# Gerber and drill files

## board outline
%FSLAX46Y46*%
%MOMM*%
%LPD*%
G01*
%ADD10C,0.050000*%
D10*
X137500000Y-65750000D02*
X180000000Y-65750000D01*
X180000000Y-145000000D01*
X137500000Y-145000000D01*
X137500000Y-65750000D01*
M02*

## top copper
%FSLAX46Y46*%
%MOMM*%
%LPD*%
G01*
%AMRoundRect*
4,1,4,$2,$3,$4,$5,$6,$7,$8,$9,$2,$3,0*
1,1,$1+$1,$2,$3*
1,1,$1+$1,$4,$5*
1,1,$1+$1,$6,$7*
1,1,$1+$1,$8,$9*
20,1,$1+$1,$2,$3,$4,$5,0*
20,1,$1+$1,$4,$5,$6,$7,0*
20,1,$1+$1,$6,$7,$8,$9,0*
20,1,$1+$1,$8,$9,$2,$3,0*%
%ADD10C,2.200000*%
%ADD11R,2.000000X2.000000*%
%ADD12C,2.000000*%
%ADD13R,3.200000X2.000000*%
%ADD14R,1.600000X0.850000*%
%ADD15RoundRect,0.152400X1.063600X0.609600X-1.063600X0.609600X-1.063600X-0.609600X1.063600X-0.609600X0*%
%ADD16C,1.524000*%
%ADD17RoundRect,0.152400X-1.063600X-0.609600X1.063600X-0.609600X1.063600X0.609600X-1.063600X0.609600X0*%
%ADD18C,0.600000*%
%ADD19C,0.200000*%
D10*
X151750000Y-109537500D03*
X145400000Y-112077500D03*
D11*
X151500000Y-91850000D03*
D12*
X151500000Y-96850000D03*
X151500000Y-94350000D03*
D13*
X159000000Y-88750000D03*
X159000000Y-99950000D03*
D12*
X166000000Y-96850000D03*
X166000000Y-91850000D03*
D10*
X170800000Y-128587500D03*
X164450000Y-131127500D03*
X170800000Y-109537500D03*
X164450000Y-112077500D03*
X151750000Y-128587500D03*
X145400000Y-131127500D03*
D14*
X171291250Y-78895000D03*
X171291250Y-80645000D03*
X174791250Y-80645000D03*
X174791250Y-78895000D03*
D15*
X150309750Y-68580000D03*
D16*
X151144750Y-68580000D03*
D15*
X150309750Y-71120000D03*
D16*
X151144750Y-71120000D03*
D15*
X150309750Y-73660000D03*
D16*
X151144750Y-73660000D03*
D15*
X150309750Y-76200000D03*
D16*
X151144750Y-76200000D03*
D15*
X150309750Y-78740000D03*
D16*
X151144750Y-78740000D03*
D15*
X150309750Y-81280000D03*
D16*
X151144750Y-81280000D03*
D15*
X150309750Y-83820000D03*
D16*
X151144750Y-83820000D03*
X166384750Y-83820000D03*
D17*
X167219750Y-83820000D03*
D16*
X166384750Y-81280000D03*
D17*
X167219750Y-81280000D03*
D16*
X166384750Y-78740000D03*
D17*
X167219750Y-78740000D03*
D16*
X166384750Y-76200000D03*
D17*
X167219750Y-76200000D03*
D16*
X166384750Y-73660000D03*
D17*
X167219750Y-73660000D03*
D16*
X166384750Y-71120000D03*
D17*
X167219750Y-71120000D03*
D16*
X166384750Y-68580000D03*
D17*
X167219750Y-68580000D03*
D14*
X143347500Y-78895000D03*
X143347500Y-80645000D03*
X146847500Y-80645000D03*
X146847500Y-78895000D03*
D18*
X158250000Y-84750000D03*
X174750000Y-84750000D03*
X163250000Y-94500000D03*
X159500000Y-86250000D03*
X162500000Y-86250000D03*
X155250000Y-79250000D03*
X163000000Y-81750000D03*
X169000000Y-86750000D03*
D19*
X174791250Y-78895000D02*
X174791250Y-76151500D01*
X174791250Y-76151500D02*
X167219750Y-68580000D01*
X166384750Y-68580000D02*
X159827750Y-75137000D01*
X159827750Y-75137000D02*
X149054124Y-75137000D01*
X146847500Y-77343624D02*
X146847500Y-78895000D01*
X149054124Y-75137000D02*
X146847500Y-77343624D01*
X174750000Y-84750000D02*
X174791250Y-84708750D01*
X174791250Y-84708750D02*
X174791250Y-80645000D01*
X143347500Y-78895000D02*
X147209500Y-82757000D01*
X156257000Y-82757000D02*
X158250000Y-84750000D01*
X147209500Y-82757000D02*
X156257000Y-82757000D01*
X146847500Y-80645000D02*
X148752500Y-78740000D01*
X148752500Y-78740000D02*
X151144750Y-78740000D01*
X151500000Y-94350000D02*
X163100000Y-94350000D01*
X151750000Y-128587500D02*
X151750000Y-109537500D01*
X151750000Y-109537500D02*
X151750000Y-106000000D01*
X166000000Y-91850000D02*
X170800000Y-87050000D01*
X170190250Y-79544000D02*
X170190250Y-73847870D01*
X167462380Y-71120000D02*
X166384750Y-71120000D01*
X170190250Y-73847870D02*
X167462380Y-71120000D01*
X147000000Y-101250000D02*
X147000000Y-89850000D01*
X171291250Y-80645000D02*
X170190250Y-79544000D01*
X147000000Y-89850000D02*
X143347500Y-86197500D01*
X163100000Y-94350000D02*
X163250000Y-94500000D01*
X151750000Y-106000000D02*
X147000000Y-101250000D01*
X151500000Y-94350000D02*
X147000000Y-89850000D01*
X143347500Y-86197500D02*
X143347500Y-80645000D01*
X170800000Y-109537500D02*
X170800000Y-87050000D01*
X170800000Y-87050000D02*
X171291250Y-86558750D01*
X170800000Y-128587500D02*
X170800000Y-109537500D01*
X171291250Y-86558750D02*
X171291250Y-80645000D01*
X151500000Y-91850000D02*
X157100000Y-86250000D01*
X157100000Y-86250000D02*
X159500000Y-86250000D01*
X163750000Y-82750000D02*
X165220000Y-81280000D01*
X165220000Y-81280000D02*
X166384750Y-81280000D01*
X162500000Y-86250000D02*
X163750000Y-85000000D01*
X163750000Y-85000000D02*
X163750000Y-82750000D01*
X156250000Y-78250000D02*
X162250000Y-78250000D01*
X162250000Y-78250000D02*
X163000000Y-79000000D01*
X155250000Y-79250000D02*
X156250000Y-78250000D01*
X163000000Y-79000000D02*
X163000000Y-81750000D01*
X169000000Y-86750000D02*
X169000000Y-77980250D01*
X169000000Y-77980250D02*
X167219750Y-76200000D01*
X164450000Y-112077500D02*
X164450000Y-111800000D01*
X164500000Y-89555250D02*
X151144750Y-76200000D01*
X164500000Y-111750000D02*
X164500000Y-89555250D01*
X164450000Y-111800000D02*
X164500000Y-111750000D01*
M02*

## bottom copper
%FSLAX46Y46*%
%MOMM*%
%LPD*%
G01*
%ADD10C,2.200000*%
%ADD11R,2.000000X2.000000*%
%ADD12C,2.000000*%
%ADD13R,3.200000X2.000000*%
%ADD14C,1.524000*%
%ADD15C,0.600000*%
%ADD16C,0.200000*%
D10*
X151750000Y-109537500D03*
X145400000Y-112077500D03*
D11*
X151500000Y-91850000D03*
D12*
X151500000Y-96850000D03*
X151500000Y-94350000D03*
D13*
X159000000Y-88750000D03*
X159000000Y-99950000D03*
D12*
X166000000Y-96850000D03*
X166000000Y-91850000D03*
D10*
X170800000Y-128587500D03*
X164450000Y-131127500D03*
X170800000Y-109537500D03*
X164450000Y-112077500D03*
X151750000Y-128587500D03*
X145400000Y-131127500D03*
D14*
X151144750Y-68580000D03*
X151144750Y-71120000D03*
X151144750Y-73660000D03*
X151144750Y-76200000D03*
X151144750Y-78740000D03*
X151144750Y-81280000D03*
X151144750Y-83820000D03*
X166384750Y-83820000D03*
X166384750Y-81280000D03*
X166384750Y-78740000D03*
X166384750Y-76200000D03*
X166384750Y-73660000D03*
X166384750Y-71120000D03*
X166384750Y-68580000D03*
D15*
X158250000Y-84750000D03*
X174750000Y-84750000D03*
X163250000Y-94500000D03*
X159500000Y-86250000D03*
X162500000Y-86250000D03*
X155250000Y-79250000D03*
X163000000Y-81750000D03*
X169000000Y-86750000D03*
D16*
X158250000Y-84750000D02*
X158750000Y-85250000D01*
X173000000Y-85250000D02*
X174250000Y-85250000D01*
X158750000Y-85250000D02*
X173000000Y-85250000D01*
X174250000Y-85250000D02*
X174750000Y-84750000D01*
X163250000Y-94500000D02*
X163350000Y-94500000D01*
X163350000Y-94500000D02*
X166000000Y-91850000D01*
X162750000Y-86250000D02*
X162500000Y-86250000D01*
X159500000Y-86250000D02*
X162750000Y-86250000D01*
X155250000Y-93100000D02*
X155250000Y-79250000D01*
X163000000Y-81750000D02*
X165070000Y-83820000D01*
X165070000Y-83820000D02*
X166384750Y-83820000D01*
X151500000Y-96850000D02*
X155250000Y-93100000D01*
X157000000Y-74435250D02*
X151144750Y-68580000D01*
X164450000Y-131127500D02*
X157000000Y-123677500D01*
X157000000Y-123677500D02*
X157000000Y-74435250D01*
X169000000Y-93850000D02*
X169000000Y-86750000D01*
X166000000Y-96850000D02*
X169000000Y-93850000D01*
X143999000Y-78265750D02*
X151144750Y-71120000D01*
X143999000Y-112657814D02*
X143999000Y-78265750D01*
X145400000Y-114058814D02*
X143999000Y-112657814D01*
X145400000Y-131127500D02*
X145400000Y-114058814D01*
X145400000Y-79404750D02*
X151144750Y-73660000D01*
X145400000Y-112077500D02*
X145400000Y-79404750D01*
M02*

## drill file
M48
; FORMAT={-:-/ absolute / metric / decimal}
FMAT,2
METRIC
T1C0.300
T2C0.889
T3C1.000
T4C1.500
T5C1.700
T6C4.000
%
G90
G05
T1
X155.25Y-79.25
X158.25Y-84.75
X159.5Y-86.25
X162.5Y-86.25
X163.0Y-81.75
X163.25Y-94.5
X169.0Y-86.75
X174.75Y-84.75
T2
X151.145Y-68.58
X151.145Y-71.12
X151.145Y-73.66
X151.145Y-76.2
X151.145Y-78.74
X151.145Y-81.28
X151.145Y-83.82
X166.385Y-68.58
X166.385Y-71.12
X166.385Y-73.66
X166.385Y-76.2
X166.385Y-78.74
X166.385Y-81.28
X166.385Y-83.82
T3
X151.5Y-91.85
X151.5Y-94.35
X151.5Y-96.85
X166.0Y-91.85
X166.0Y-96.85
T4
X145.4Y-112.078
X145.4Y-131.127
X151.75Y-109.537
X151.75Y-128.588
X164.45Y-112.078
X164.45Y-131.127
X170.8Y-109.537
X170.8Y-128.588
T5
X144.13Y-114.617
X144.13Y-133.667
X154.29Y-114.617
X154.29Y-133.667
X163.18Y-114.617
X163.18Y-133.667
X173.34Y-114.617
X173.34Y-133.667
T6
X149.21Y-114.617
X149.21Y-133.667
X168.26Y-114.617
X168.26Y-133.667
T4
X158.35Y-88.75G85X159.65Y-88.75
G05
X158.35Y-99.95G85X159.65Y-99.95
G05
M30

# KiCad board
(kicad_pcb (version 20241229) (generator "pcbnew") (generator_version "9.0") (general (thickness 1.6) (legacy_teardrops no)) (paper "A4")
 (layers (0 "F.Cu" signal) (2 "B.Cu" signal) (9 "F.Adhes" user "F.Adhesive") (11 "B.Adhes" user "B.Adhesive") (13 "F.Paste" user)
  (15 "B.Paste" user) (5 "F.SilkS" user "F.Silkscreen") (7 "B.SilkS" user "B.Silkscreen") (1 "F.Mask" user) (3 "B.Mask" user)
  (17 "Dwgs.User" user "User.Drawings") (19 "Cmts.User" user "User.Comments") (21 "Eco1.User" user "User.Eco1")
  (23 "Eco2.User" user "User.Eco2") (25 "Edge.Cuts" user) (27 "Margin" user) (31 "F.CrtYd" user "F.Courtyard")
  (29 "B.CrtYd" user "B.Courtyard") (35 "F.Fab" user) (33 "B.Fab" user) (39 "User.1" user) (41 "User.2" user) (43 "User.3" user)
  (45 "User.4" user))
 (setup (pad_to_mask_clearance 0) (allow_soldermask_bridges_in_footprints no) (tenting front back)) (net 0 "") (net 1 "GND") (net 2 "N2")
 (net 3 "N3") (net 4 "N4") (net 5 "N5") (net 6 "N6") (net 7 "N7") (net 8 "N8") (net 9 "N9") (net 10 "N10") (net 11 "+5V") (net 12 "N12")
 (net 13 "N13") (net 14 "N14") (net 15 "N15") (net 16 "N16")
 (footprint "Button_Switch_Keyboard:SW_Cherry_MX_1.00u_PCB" (layer "F.Cu") (at 151.75 109.5375)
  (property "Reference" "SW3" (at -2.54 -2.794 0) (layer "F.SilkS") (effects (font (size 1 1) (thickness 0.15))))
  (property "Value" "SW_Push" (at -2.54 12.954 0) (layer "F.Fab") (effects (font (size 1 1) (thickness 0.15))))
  (pad "" np_thru_hole circle (at -7.62 5.08) (size 1.7 1.7) (drill 1.7) (layers "*.Cu" "*.Mask"))
  (pad "" np_thru_hole circle (at -2.54 5.08) (size 4 4) (drill 4) (layers "*.Cu" "*.Mask"))
  (pad "" np_thru_hole circle (at 2.54 5.08) (size 1.7 1.7) (drill 1.7) (layers "*.Cu" "*.Mask"))
  (pad "1" thru_hole circle (at 0 0) (size 2.2 2.2) (drill 1.5) (layers "*.Cu" "*.Mask") (remove_unused_layers no) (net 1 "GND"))
  (pad "2" thru_hole circle (at -6.35 2.54) (size 2.2 2.2) (drill 1.5) (layers "*.Cu" "*.Mask") (remove_unused_layers no) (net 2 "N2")))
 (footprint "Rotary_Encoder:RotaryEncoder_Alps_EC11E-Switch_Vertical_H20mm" (layer "F.Cu") (at 151.5 91.85)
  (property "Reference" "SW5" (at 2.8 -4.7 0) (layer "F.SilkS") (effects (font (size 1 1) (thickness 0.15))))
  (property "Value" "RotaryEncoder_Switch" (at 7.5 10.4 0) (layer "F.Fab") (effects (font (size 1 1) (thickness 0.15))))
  (pad "A" thru_hole rect (at 0 0) (size 2 2) (drill 1) (layers "*.Cu" "*.Mask") (remove_unused_layers no) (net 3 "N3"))
  (pad "B" thru_hole circle (at 0 5) (size 2 2) (drill 1) (layers "*.Cu" "*.Mask") (remove_unused_layers no) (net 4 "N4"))
  (pad "C" thru_hole circle (at 0 2.5) (size 2 2) (drill 1) (layers "*.Cu" "*.Mask") (remove_unused_layers no) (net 1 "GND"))
  (pad "MP" thru_hole rect (at 7.5 -3.1) (size 3.2 2) (drill oval 2.8 1.5) (layers "*.Cu" "*.Mask") (remove_unused_layers no))
  (pad "MP" thru_hole rect (at 7.5 8.1) (size 3.2 2) (drill oval 2.8 1.5) (layers "*.Cu" "*.Mask") (remove_unused_layers no))
  (pad "S1" thru_hole circle (at 14.5 5) (size 2 2) (drill 1) (layers "*.Cu" "*.Mask") (remove_unused_layers no) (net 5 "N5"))
  (pad "S2" thru_hole circle (at 14.5 0) (size 2 2) (drill 1) (layers "*.Cu" "*.Mask") (remove_unused_layers no) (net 1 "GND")))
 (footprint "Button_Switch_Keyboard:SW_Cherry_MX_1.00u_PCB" (layer "F.Cu") (at 170.8 128.5875)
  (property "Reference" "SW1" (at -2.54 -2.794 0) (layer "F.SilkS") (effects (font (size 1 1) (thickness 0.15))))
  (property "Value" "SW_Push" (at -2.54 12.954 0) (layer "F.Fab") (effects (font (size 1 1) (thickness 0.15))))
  (pad "" np_thru_hole circle (at -7.62 5.08) (size 1.7 1.7) (drill 1.7) (layers "*.Cu" "*.Mask"))
  (pad "" np_thru_hole circle (at -2.54 5.08) (size 4 4) (drill 4) (layers "*.Cu" "*.Mask"))
  (pad "" np_thru_hole circle (at 2.54 5.08) (size 1.7 1.7) (drill 1.7) (layers "*.Cu" "*.Mask"))
  (pad "1" thru_hole circle (at 0 0) (size 2.2 2.2) (drill 1.5) (layers "*.Cu" "*.Mask") (remove_unused_layers no) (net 1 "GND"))
  (pad "2" thru_hole circle (at -6.35 2.54) (size 2.2 2.2) (drill 1.5) (layers "*.Cu" "*.Mask") (remove_unused_layers no) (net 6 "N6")))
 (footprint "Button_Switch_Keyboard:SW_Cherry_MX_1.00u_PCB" (layer "F.Cu") (at 170.8 109.5375)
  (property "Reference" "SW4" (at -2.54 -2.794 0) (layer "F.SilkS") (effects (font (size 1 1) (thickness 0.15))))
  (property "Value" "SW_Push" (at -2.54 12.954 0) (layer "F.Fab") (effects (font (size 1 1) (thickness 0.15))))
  (pad "" np_thru_hole circle (at -7.62 5.08) (size 1.7 1.7) (drill 1.7) (layers "*.Cu" "*.Mask"))
  (pad "" np_thru_hole circle (at -2.54 5.08) (size 4 4) (drill 4) (layers "*.Cu" "*.Mask"))
  (pad "" np_thru_hole circle (at 2.54 5.08) (size 1.7 1.7) (drill 1.7) (layers "*.Cu" "*.Mask"))
  (pad "1" thru_hole circle (at 0 0) (size 2.2 2.2) (drill 1.5) (layers "*.Cu" "*.Mask") (remove_unused_layers no) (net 1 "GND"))
  (pad "2" thru_hole circle (at -6.35 2.54) (size 2.2 2.2) (drill 1.5) (layers "*.Cu" "*.Mask") (remove_unused_layers no) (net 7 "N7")))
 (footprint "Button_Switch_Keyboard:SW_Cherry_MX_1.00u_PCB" (layer "F.Cu") (at 151.75 128.5875)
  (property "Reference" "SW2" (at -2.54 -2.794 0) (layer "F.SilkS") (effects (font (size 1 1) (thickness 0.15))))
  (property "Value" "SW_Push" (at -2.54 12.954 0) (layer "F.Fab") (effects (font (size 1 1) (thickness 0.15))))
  (pad "" np_thru_hole circle (at -7.62 5.08) (size 1.7 1.7) (drill 1.7) (layers "*.Cu" "*.Mask"))
  (pad "" np_thru_hole circle (at -2.54 5.08) (size 4 4) (drill 4) (layers "*.Cu" "*.Mask"))
  (pad "" np_thru_hole circle (at 2.54 5.08) (size 1.7 1.7) (drill 1.7) (layers "*.Cu" "*.Mask"))
  (pad "1" thru_hole circle (at 0 0) (size 2.2 2.2) (drill 1.5) (layers "*.Cu" "*.Mask") (remove_unused_layers no) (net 1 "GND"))
  (pad "2" thru_hole circle (at -6.35 2.54) (size 2.2 2.2) (drill 1.5) (layers "*.Cu" "*.Mask") (remove_unused_layers no) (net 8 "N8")))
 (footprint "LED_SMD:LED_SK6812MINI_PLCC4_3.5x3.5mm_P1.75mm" (layer "F.Cu") (at 173.04125 79.77)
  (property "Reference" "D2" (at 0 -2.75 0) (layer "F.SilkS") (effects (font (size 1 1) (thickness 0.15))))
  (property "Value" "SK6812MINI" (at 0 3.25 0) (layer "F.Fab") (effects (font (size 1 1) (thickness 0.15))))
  (pad "1" smd rect (at -1.75 -0.875) (size 1.6 0.85) (layers "F.Cu" "F.Mask" "F.Paste") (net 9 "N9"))
  (pad "2" smd rect (at -1.75 0.875) (size 1.6 0.85) (layers "F.Cu" "F.Mask" "F.Paste") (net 1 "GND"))
  (pad "3" smd rect (at 1.75 0.875) (size 1.6 0.85) (layers "F.Cu" "F.Mask" "F.Paste") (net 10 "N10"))
  (pad "4" smd rect (at 1.75 -0.875) (size 1.6 0.85) (layers "F.Cu" "F.Mask" "F.Paste") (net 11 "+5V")))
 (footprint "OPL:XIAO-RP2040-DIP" (layer "F.Cu") (at 158.76475 76.2)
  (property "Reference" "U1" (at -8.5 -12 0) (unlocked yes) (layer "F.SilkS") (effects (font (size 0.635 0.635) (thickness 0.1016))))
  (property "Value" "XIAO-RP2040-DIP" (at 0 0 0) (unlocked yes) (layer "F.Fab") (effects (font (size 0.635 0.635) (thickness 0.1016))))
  (pad "1" smd roundrect (at -8.455 -7.62 180) (size 2.432 1.524) (layers "F.Cu" "F.Mask") (roundrect_rratio 0.1) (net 6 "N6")
   (thermal_bridge_angle 45))
  (pad "1" thru_hole circle (at -7.62 -7.62 180) (size 1.524 1.524) (drill 0.889) (layers "*.Cu" "*.Mask") (remove_unused_layers no)
   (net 6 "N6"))
  (pad "2" smd roundrect (at -8.455 -5.08 180) (size 2.432 1.524) (layers "F.Cu" "F.Mask") (roundrect_rratio 0.1) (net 8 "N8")
   (thermal_bridge_angle 45))
  (pad "2" thru_hole circle (at -7.62 -5.08 180) (size 1.524 1.524) (drill 0.889) (layers "*.Cu" "*.Mask") (remove_unused_layers no)
   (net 8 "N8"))
  (pad "3" smd roundrect (at -8.455 -2.54 180) (size 2.432 1.524) (layers "F.Cu" "F.Mask") (roundrect_rratio 0.1) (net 2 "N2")
   (thermal_bridge_angle 45))
  (pad "3" thru_hole circle (at -7.62 -2.54 180) (size 1.524 1.524) (drill 0.889) (layers "*.Cu" "*.Mask") (remove_unused_layers no)
   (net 2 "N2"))
  (pad "4" smd roundrect (at -8.455 0 180) (size 2.432 1.524) (layers "F.Cu" "F.Mask") (roundrect_rratio 0.1) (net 7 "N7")
   (thermal_bridge_angle 45))
  (pad "4" thru_hole circle (at -7.62 0 180) (size 1.524 1.524) (drill 0.889) (layers "*.Cu" "*.Mask") (remove_unused_layers no)
   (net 7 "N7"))
  (pad "5" smd roundrect (at -8.455 2.54 180) (size 2.432 1.524) (layers "F.Cu" "F.Mask") (roundrect_rratio 0.1) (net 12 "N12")
   (thermal_bridge_angle 45))
  (pad "5" thru_hole circle (at -7.62 2.54 180) (size 1.524 1.524) (drill 0.889) (layers "*.Cu" "*.Mask") (remove_unused_layers no)
   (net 12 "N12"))
  (pad "6" smd roundrect (at -8.455 5.08 180) (size 2.432 1.524) (layers "F.Cu" "F.Mask") (roundrect_rratio 0.1) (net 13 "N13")
   (thermal_bridge_angle 45))
  (pad "6" thru_hole circle (at -7.62 5.08 180) (size 1.524 1.524) (drill 0.889) (layers "*.Cu" "*.Mask") (remove_unused_layers no)
   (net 13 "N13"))
  (pad "7" smd roundrect (at -8.455 7.62 180) (size 2.432 1.524) (layers "F.Cu" "F.Mask") (roundrect_rratio 0.1) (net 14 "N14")
   (thermal_bridge_angle 45))
  (pad "7" thru_hole circle (at -7.62 7.62 180) (size 1.524 1.524) (drill 0.889) (layers "*.Cu" "*.Mask") (remove_unused_layers no)
   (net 14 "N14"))
  (pad "8" thru_hole circle (at 7.62 7.62) (size 1.524 1.524) (drill 0.889) (layers "*.Cu" "*.Mask") (remove_unused_layers no) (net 4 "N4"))
  (pad "8" smd roundrect (at 8.455 7.62) (size 2.432 1.524) (layers "F.Cu" "F.Mask") (roundrect_rratio 0.1) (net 4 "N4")
   (thermal_bridge_angle 45))
  (pad "9" thru_hole circle (at 7.62 5.08) (size 1.524 1.524) (drill 0.889) (layers "*.Cu" "*.Mask") (remove_unused_layers no) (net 3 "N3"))
  (pad "9" smd roundrect (at 8.455 5.08) (size 2.432 1.524) (layers "F.Cu" "F.Mask") (roundrect_rratio 0.1) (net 3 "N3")
   (thermal_bridge_angle 45))
  (pad "10" thru_hole circle (at 7.62 2.54) (size 1.524 1.524) (drill 0.889) (layers "*.Cu" "*.Mask") (remove_unused_layers no)
   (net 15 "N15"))
  (pad "10" smd roundrect (at 8.455 2.54) (size 2.432 1.524) (layers "F.Cu" "F.Mask") (roundrect_rratio 0.1) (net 15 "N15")
   (thermal_bridge_angle 45))
  (pad "11" thru_hole circle (at 7.62 0) (size 1.524 1.524) (drill 0.889) (layers "*.Cu" "*.Mask") (remove_unused_layers no) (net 5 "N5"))
  (pad "11" smd roundrect (at 8.455 0) (size 2.432 1.524) (layers "F.Cu" "F.Mask") (roundrect_rratio 0.1) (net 5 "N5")
   (thermal_bridge_angle 45))
  (pad "12" thru_hole circle (at 7.62 -2.54) (size 1.524 1.524) (drill 0.889) (layers "*.Cu" "*.Mask") (remove_unused_layers no)
   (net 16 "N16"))
  (pad "12" smd roundrect (at 8.455 -2.54) (size 2.432 1.524) (layers "F.Cu" "F.Mask") (roundrect_rratio 0.1) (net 16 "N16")
   (thermal_bridge_angle 45))
  (pad "13" thru_hole circle (at 7.62 -5.08) (size 1.524 1.524) (drill 0.889) (layers "*.Cu" "*.Mask") (remove_unused_layers no)
   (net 1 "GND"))
  (pad "13" smd roundrect (at 8.455 -5.08) (size 2.432 1.524) (layers "F.Cu" "F.Mask") (roundrect_rratio 0.1) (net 1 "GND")
   (thermal_bridge_angle 45))
  (pad "14" thru_hole circle (at 7.62 -7.62) (size 1.524 1.524) (drill 0.889) (layers "*.Cu" "*.Mask") (remove_unused_layers no)
   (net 11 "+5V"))
  (pad "14" smd roundrect (at 8.455 -7.62) (size 2.432 1.524) (layers "F.Cu" "F.Mask") (roundrect_rratio 0.1) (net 11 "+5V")
   (thermal_bridge_angle 45)))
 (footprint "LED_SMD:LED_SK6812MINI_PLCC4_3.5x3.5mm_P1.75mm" (layer "F.Cu") (at 145.0975 79.77)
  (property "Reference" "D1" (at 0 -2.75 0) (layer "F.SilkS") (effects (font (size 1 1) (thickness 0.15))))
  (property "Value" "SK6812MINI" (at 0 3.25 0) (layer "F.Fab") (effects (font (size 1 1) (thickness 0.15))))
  (pad "1" smd rect (at -1.75 -0.875) (size 1.6 0.85) (layers "F.Cu" "F.Mask" "F.Paste") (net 10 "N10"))
  (pad "2" smd rect (at -1.75 0.875) (size 1.6 0.85) (layers "F.Cu" "F.Mask" "F.Paste") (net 1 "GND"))
  (pad "3" smd rect (at 1.75 0.875) (size 1.6 0.85) (layers "F.Cu" "F.Mask" "F.Paste") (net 12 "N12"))
  (pad "4" smd rect (at 1.75 -0.875) (size 1.6 0.85) (layers "F.Cu" "F.Mask" "F.Paste") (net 11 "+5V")))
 (gr_rect (start 137.5 65.75) (end 180 145) (stroke (width 0.05) (type default)) (fill no) (layer "Edge.Cuts"))
 (segment (start 174.79125 78.895) (end 174.79125 76.1515) (width 0.2) (layer "F.Cu") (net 11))
 (segment (start 174.79125 76.1515) (end 167.21975 68.58) (width 0.2) (layer "F.Cu") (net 11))
 (segment (start 166.38475 68.58) (end 159.82775 75.137) (width 0.2) (layer "F.Cu") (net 11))
 (segment (start 159.82775 75.137) (end 149.054124 75.137) (width 0.2) (layer "F.Cu") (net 11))
 (segment (start 146.8475 77.343624) (end 146.8475 78.895) (width 0.2) (layer "F.Cu") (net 11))
 (segment (start 149.054124 75.137) (end 146.8475 77.343624) (width 0.2) (layer "F.Cu") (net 11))
 (segment (start 174.75 84.75) (end 174.79125 84.70875) (width 0.2) (layer "F.Cu") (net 10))
 (segment (start 174.79125 84.70875) (end 174.79125 80.645) (width 0.2) (layer "F.Cu") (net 10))
 (segment (start 143.3475 78.895) (end 147.2095 82.757) (width 0.2) (layer "F.Cu") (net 10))
 (segment (start 156.257 82.757) (end 158.25 84.75) (width 0.2) (layer "F.Cu") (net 10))
 (segment (start 147.2095 82.757) (end 156.257 82.757) (width 0.2) (layer "F.Cu") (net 10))
 (via (at 158.25 84.75) (size 0.6) (drill 0.3) (layers "F.Cu" "B.Cu") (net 10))
 (via (at 174.75 84.75) (size 0.6) (drill 0.3) (layers "F.Cu" "B.Cu") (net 10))
 (segment (start 158.25 84.75) (end 158.75 85.25) (width 0.2) (layer "B.Cu") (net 10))
 (segment (start 173 85.25) (end 174.25 85.25) (width 0.2) (layer "B.Cu") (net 10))
 (segment (start 158.75 85.25) (end 173 85.25) (width 0.2) (layer "B.Cu") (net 10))
 (segment (start 174.25 85.25) (end 174.75 84.75) (width 0.2) (layer "B.Cu") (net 10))
 (segment (start 146.8475 80.645) (end 148.7525 78.74) (width 0.2) (layer "F.Cu") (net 12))
 (segment (start 148.7525 78.74) (end 151.14475 78.74) (width 0.2) (layer "F.Cu") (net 12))
 (segment (start 151.5 94.35) (end 163.1 94.35) (width 0.2) (layer "F.Cu") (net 1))
 (segment (start 151.75 128.5875) (end 151.75 109.5375) (width 0.2) (layer "F.Cu") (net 1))
 (segment (start 151.75 109.5375) (end 151.75 106) (width 0.2) (layer "F.Cu") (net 1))
 (segment (start 166 91.85) (end 170.8 87.05) (width 0.2) (layer "F.Cu") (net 1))
 (segment (start 170.19025 79.544) (end 170.19025 73.84787) (width 0.2) (layer "F.Cu") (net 1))
 (segment (start 167.46238 71.12) (end 166.38475 71.12) (width 0.2) (layer "F.Cu") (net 1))
 (segment (start 170.19025 73.84787) (end 167.46238 71.12) (width 0.2) (layer "F.Cu") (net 1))
 (segment (start 147 101.25) (end 147 89.85) (width 0.2) (layer "F.Cu") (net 1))
 (segment (start 171.29125 80.645) (end 170.19025 79.544) (width 0.2) (layer "F.Cu") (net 1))
 (segment (start 147 89.85) (end 143.3475 86.1975) (width 0.2) (layer "F.Cu") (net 1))
 (segment (start 163.1 94.35) (end 163.25 94.5) (width 0.2) (layer "F.Cu") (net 1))
 (segment (start 151.75 106) (end 147 101.25) (width 0.2) (layer "F.Cu") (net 1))
 (segment (start 151.5 94.35) (end 147 89.85) (width 0.2) (layer "F.Cu") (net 1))
 (segment (start 143.3475 86.1975) (end 143.3475 80.645) (width 0.2) (layer "F.Cu") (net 1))
 (segment (start 170.8 109.5375) (end 170.8 87.05) (width 0.2) (layer "F.Cu") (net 1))
 (segment (start 170.8 87.05) (end 171.29125 86.55875) (width 0.2) (layer "F.Cu") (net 1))
 (segment (start 170.8 128.5875) (end 170.8 109.5375) (width 0.2) (layer "F.Cu") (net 1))
 (segment (start 171.29125 86.55875) (end 171.29125 80.645) (width 0.2) (layer "F.Cu") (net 1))
 (via (at 163.25 94.5) (size 0.6) (drill 0.3) (layers "F.Cu" "B.Cu") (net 1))
 (segment (start 163.25 94.5) (end 163.35 94.5) (width 0.2) (layer "B.Cu") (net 1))
 (segment (start 163.35 94.5) (end 166 91.85) (width 0.2) (layer "B.Cu") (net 1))
 (segment (start 151.5 91.85) (end 157.1 86.25) (width 0.2) (layer "F.Cu") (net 3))
 (segment (start 157.1 86.25) (end 159.5 86.25) (width 0.2) (layer "F.Cu") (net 3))
 (segment (start 163.75 82.75) (end 165.22 81.28) (width 0.2) (layer "F.Cu") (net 3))
 (segment (start 165.22 81.28) (end 166.38475 81.28) (width 0.2) (layer "F.Cu") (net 3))
 (segment (start 162.5 86.25) (end 163.75 85) (width 0.2) (layer "F.Cu") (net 3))
 (segment (start 163.75 85) (end 163.75 82.75) (width 0.2) (layer "F.Cu") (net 3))
 (via (at 159.5 86.25) (size 0.6) (drill 0.3) (layers "F.Cu" "B.Cu") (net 3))
 (via (at 162.5 86.25) (size 0.6) (drill 0.3) (layers "F.Cu" "B.Cu") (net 3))
 (segment (start 162.75 86.25) (end 162.5 86.25) (width 0.2) (layer "B.Cu") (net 3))
 (segment (start 159.5 86.25) (end 162.75 86.25) (width 0.2) (layer "B.Cu") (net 3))
 (segment (start 156.25 78.25) (end 162.25 78.25) (width 0.2) (layer "F.Cu") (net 4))
 (segment (start 162.25 78.25) (end 163 79) (width 0.2) (layer "F.Cu") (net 4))
 (segment (start 155.25 79.25) (end 156.25 78.25) (width 0.2) (layer "F.Cu") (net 4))
 (segment (start 163 79) (end 163 81.75) (width 0.2) (layer "F.Cu") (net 4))
 (via (at 155.25 79.25) (size 0.6) (drill 0.3) (layers "F.Cu" "B.Cu") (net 4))
 (via (at 163 81.75) (size 0.6) (drill 0.3) (layers "F.Cu" "B.Cu") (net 4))
 (segment (start 155.25 93.1) (end 155.25 79.25) (width 0.2) (layer "B.Cu") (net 4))
 (segment (start 163 81.75) (end 165.07 83.82) (width 0.2) (layer "B.Cu") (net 4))
 (segment (start 165.07 83.82) (end 166.38475 83.82) (width 0.2) (layer "B.Cu") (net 4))
 (segment (start 151.5 96.85) (end 155.25 93.1) (width 0.2) (layer "B.Cu") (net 4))
 (segment (start 157 74.43525) (end 151.14475 68.58) (width 0.2) (layer "B.Cu") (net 6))
 (segment (start 164.45 131.1275) (end 157 123.6775) (width 0.2) (layer "B.Cu") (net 6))
 (segment (start 157 123.6775) (end 157 74.43525) (width 0.2) (layer "B.Cu") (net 6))
 (segment (start 169 86.75) (end 169 77.98025) (width 0.2) (layer "F.Cu") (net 5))
 (segment (start 169 77.98025) (end 167.21975 76.2) (width 0.2) (layer "F.Cu") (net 5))
 (via (at 169 86.75) (size 0.6) (drill 0.3) (layers "F.Cu" "B.Cu") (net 5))
 (segment (start 169 93.85) (end 169 86.75) (width 0.2) (layer "B.Cu") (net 5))
 (segment (start 166 96.85) (end 169 93.85) (width 0.2) (layer "B.Cu") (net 5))
 (segment (start 143.999 78.26575) (end 151.14475 71.12) (width 0.2) (layer "B.Cu") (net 8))
 (segment (start 143.999 112.657814) (end 143.999 78.26575) (width 0.2) (layer "B.Cu") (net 8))
 (segment (start 145.4 114.058814) (end 143.999 112.657814) (width 0.2) (layer "B.Cu") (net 8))
 (segment (start 145.4 131.1275) (end 145.4 114.058814) (width 0.2) (layer "B.Cu") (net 8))
 (segment (start 145.4 79.40475) (end 151.14475 73.66) (width 0.2) (layer "B.Cu") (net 2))
 (segment (start 145.4 112.0775) (end 145.4 79.40475) (width 0.2) (layer "B.Cu") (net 2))
 (segment (start 164.45 112.0775) (end 164.45 111.8) (width 0.2) (layer "F.Cu") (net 7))
 (segment (start 164.5 89.55525) (end 151.14475 76.2) (width 0.2) (layer "F.Cu") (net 7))
 (segment (start 164.5 111.75) (end 164.5 89.55525) (width 0.2) (layer "F.Cu") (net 7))
 (segment (start 164.45 111.8) (end 164.5 111.75) (width 0.2) (layer "F.Cu") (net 7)))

